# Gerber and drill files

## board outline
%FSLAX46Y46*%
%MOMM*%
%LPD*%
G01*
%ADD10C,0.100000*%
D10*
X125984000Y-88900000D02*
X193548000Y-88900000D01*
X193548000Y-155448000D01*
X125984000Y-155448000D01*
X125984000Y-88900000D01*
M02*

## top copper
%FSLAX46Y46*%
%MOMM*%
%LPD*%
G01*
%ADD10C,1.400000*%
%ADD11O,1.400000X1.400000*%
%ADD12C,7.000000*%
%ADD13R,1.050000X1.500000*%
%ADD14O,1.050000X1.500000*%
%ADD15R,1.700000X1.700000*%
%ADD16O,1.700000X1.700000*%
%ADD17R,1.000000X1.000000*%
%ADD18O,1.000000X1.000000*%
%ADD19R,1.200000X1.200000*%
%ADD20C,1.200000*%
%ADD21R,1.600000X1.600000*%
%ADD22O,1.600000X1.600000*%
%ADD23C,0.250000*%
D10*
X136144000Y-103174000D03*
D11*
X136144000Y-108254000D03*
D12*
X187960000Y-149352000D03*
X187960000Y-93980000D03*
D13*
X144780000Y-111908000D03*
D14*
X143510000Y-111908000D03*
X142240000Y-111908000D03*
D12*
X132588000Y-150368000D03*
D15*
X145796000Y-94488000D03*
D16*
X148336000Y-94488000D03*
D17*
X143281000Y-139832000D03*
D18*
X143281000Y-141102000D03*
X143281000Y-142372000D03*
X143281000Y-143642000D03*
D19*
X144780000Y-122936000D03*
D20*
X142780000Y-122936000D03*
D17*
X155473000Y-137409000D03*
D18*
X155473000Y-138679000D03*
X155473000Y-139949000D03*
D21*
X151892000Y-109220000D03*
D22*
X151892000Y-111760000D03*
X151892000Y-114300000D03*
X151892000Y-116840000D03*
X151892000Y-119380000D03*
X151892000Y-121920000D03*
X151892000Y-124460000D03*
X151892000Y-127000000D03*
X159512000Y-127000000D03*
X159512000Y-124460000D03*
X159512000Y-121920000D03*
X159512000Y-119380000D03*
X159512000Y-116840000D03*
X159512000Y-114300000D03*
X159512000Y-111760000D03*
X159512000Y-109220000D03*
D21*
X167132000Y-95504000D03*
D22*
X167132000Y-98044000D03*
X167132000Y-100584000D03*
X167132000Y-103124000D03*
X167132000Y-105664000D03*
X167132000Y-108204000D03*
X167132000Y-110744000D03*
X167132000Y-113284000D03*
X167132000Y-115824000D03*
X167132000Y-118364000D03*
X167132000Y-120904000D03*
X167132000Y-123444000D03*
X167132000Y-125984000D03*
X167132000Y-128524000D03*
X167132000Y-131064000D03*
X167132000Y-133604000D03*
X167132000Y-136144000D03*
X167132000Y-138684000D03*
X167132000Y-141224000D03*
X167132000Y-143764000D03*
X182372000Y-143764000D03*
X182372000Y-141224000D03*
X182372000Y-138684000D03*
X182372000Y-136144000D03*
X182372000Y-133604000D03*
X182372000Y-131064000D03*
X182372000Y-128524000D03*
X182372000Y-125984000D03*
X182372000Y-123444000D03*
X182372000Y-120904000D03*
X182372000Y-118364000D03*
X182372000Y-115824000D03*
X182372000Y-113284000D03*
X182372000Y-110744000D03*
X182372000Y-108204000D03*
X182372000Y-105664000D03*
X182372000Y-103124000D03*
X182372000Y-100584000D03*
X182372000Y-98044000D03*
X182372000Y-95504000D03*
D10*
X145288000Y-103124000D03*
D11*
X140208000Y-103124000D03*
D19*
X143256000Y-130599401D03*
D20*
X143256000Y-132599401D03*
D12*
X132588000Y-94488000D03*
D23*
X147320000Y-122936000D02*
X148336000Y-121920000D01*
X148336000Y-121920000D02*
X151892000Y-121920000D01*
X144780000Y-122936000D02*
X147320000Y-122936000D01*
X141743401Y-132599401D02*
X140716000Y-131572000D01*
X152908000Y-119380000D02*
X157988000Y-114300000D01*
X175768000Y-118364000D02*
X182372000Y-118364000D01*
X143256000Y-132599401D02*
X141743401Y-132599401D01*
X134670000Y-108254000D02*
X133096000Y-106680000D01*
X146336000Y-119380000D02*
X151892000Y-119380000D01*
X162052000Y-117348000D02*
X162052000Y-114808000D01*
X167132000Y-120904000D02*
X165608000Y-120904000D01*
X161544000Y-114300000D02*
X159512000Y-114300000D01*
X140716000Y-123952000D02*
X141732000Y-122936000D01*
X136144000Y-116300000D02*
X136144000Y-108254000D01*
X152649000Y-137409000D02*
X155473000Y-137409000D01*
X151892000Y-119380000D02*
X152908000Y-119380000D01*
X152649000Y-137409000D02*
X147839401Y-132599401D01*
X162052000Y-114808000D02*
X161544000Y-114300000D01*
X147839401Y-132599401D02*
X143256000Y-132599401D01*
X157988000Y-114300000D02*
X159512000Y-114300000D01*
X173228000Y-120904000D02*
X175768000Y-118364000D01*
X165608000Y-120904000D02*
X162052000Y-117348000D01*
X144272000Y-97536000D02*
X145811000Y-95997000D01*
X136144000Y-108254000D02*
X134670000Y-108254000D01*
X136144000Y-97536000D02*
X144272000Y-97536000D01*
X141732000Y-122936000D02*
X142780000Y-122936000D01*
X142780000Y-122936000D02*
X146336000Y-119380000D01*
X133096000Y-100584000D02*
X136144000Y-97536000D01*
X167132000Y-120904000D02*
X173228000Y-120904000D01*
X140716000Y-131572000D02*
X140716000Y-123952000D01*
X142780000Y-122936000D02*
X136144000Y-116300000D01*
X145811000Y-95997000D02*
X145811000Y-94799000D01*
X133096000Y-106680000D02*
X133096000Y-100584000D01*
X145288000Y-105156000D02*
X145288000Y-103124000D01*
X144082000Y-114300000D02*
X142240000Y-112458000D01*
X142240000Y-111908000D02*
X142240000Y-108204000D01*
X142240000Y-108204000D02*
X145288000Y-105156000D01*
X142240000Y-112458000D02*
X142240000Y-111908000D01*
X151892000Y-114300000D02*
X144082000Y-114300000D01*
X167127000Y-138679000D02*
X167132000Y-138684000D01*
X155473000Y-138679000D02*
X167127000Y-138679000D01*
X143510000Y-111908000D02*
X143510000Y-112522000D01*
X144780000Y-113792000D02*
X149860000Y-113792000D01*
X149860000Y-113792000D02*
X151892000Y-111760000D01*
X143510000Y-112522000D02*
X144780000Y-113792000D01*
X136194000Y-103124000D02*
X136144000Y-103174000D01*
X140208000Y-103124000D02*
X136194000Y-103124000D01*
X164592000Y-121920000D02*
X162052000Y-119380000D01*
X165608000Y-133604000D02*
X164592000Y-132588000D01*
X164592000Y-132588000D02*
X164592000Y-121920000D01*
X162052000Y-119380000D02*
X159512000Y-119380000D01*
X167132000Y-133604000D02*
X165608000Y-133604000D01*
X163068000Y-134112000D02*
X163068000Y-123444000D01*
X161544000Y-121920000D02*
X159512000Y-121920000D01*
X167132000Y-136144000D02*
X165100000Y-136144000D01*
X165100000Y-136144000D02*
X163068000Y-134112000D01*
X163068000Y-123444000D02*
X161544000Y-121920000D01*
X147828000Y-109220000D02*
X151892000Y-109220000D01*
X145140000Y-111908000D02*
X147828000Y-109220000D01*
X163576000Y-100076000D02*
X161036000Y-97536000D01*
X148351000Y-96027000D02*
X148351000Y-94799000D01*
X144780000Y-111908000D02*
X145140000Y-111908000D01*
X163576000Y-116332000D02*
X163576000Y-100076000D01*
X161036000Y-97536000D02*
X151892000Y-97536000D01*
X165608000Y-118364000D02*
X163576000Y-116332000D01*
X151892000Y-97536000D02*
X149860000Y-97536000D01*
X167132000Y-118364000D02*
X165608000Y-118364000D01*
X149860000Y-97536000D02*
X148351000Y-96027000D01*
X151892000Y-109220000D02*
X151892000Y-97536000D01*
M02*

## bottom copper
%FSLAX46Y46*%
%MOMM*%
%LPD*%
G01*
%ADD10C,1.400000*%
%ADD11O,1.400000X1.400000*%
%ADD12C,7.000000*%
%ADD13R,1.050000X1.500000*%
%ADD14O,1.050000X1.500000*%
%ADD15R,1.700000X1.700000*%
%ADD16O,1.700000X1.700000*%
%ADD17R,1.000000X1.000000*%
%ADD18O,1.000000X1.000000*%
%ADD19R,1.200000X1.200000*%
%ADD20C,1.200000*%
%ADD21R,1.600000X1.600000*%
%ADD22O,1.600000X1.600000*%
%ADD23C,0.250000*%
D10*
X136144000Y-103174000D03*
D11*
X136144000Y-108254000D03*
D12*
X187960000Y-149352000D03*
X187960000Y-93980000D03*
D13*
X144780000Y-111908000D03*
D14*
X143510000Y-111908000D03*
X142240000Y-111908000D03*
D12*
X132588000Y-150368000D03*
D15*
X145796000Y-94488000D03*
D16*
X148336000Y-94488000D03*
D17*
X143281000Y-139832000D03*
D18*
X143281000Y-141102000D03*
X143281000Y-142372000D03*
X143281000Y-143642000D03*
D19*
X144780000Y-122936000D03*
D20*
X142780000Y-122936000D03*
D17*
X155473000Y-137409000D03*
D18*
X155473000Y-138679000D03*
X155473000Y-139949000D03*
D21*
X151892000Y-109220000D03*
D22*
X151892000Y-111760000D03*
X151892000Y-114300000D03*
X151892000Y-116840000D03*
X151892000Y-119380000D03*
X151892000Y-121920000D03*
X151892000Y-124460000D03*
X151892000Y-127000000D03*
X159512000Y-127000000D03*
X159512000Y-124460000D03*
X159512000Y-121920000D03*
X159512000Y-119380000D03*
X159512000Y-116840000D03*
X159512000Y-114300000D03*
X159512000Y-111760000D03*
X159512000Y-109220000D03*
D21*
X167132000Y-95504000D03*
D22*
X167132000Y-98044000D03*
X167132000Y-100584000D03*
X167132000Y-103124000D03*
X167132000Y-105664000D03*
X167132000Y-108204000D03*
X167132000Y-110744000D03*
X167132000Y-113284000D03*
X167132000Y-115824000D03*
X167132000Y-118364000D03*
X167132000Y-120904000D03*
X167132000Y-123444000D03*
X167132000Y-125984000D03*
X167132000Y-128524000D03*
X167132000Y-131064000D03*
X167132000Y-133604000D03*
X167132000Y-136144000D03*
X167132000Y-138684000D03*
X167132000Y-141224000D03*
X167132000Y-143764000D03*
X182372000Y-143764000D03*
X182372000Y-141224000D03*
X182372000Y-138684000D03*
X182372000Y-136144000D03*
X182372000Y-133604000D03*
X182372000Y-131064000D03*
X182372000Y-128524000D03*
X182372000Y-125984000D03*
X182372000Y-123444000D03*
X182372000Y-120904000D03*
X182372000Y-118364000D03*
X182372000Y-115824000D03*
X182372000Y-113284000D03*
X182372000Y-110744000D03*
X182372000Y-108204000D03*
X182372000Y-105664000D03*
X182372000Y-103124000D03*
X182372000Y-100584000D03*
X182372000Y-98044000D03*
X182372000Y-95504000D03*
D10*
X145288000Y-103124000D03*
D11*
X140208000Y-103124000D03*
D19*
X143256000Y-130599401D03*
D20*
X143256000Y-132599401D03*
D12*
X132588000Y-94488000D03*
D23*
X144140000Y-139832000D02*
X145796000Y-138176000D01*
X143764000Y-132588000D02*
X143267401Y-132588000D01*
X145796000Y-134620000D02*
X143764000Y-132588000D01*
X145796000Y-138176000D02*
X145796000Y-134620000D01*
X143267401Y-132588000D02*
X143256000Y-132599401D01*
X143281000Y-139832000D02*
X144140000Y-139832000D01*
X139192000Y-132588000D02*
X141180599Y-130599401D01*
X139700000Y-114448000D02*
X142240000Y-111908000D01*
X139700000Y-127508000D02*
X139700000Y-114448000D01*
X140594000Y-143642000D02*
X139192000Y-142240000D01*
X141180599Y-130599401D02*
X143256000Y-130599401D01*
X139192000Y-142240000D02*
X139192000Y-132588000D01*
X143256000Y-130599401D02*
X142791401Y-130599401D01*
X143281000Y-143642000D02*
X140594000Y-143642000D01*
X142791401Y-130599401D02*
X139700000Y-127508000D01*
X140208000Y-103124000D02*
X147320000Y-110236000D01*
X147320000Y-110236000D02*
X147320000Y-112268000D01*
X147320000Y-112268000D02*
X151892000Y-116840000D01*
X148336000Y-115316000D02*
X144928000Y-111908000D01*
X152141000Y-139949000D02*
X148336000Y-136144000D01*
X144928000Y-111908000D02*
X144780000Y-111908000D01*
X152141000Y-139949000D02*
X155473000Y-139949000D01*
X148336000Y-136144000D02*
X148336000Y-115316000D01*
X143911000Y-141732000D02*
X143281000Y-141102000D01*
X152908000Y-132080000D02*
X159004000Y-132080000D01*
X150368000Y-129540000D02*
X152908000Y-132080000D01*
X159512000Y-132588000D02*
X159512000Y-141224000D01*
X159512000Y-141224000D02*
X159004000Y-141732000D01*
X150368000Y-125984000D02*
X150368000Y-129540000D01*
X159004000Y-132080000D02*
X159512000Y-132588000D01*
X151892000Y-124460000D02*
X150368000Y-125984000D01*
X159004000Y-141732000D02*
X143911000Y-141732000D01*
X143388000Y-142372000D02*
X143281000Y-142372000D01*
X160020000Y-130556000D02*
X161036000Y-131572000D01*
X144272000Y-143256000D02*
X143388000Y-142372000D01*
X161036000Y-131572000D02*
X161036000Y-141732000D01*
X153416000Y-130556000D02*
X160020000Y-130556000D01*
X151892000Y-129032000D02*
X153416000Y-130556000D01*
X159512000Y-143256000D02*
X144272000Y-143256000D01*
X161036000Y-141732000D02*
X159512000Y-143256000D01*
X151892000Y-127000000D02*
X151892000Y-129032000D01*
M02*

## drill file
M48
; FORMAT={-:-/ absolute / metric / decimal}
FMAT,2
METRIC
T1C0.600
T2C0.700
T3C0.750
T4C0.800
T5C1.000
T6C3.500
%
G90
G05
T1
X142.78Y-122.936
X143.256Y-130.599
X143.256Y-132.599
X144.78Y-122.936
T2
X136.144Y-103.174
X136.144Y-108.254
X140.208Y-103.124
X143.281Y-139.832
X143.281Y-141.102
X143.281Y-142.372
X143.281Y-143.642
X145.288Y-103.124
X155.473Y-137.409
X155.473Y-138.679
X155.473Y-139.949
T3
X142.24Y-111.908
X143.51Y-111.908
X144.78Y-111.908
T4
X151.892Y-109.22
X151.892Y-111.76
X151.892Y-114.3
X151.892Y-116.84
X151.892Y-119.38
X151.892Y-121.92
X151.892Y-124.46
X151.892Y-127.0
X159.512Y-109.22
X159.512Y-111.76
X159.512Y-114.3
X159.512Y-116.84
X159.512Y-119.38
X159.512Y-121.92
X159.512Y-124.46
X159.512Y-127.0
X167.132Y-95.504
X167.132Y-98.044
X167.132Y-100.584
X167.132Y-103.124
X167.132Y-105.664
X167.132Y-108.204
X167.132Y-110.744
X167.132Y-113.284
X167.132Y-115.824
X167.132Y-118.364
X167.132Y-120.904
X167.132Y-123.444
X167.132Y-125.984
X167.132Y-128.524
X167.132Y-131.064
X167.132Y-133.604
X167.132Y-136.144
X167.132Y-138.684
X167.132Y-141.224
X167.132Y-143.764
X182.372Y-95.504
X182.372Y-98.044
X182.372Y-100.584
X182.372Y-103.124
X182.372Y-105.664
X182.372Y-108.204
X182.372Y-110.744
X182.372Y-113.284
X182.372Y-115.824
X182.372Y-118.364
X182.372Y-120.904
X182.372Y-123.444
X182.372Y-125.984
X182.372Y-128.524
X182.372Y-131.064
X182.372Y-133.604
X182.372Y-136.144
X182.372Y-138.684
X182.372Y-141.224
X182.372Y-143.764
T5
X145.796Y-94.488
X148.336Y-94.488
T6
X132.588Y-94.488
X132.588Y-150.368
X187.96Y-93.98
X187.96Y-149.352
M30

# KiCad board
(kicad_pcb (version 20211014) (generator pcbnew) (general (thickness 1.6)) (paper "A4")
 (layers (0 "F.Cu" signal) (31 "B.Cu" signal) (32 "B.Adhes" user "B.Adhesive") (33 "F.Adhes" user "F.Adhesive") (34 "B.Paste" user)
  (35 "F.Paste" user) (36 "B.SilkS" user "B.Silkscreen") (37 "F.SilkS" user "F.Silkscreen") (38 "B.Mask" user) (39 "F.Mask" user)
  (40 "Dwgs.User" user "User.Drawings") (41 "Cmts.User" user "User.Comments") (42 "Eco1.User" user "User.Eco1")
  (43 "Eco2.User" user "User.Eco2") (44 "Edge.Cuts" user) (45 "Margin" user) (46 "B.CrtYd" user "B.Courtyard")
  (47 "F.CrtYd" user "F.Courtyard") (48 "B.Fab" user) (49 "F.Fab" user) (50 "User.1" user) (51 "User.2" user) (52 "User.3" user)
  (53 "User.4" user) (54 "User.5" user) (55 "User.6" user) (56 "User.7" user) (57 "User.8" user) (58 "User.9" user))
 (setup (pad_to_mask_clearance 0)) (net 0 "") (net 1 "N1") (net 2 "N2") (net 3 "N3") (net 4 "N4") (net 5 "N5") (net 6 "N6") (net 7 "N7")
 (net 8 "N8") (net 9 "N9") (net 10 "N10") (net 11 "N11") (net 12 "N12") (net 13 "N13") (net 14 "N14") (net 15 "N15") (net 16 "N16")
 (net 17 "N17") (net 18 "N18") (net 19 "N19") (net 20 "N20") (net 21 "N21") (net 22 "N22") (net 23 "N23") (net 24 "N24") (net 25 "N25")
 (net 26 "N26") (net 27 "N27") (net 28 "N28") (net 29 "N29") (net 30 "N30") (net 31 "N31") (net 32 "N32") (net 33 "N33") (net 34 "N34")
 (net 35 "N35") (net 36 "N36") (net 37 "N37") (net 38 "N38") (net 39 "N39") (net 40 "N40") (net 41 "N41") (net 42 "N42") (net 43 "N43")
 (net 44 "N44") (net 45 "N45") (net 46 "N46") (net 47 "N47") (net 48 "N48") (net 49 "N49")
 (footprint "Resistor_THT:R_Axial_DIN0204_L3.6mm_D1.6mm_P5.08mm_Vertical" (layer "F.Cu") (at 136.144 103.174 -90)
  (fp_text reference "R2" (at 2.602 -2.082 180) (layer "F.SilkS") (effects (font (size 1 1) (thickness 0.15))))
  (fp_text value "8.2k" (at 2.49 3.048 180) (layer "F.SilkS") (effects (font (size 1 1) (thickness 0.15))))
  (pad "1" thru_hole circle (at 0 0 270) (size 1.4 1.4) (drill 0.7) (layers *.Cu *.Mask) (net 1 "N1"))
  (pad "2" thru_hole oval (at 5.08 0 270) (size 1.4 1.4) (drill 0.7) (layers *.Cu *.Mask) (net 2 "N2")))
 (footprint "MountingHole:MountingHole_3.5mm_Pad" (layer "F.Cu") (at 187.96 149.352)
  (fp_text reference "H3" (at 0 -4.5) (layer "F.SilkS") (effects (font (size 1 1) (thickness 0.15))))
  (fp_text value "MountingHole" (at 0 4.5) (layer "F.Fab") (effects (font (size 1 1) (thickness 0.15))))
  (pad "1" thru_hole circle (at 0 0) (size 7 7) (drill 3.5) (layers *.Cu *.Mask)))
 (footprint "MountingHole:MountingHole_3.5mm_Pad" (layer "F.Cu") (at 187.96 93.98)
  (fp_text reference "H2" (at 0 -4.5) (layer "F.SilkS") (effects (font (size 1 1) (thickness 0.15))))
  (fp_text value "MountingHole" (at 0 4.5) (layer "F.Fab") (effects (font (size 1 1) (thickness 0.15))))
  (pad "1" thru_hole circle (at 0 0) (size 7 7) (drill 3.5) (layers *.Cu *.Mask)))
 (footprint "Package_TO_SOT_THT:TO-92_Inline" (layer "F.Cu") (at 144.78 111.908 180)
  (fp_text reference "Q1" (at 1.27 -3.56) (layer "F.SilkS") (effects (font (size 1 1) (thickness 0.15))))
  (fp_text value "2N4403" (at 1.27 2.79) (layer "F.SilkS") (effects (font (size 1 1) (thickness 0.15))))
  (pad "1" thru_hole rect (at 0 0 180) (size 1.05 1.5) (drill 0.75) (layers *.Cu *.Mask) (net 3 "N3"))
  (pad "2" thru_hole oval (at 1.27 0 180) (size 1.05 1.5) (drill 0.75) (layers *.Cu *.Mask) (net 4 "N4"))
  (pad "3" thru_hole oval (at 2.54 0 180) (size 1.05 1.5) (drill 0.75) (layers *.Cu *.Mask) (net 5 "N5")))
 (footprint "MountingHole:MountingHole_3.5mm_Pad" (layer "F.Cu") (at 132.588 150.368)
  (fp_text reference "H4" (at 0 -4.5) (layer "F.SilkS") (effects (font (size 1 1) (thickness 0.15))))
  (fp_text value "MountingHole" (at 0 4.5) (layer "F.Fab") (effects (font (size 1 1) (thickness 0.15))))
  (pad "1" thru_hole circle (at 0 0) (size 7 7) (drill 3.5) (layers *.Cu *.Mask)))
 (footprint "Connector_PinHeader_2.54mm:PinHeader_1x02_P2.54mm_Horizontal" (layer "F.Cu") (at 145.796 94.488 90)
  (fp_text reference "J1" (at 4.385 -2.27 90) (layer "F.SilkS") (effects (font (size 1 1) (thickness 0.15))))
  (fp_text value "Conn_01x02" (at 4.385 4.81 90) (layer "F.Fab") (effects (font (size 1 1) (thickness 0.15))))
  (pad "1" thru_hole rect (at 0 0 90) (size 1.7 1.7) (drill 1) (layers *.Cu *.Mask) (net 2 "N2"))
  (pad "2" thru_hole oval (at 0 2.54 90) (size 1.7 1.7) (drill 1) (layers *.Cu *.Mask) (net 3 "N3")))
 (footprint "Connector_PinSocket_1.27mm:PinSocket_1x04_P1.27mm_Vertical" (layer "F.Cu") (at 143.281 139.832)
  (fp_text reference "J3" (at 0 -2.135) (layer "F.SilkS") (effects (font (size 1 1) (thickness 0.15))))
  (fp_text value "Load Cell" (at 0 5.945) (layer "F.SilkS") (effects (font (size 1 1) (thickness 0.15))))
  (pad "1" thru_hole rect (at 0 0) (size 1 1) (drill 0.7) (layers *.Cu *.Mask) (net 2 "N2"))
  (pad "2" thru_hole oval (at 0 1.27) (size 1 1) (drill 0.7) (layers *.Cu *.Mask) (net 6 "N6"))
  (pad "3" thru_hole oval (at 0 2.54) (size 1 1) (drill 0.7) (layers *.Cu *.Mask) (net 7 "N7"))
  (pad "4" thru_hole oval (at 0 3.81) (size 1 1) (drill 0.7) (layers *.Cu *.Mask) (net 5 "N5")))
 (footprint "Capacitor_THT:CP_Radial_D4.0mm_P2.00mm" (layer "F.Cu") (at 144.78 122.936 180)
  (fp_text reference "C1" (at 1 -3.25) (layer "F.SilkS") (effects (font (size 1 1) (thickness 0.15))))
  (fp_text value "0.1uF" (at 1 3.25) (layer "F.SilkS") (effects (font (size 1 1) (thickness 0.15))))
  (pad "1" thru_hole rect (at 0 0 180) (size 1.2 1.2) (drill 0.6) (layers *.Cu *.Mask) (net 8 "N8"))
  (pad "2" thru_hole circle (at 2 0 180) (size 1.2 1.2) (drill 0.6) (layers *.Cu *.Mask) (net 2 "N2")))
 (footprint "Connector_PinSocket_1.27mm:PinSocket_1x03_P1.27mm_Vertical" (layer "F.Cu") (at 155.473 137.409)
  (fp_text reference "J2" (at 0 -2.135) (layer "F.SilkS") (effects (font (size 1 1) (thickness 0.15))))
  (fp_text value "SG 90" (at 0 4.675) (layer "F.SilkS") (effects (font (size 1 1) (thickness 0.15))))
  (pad "1" thru_hole rect (at 0 0) (size 1 1) (drill 0.7) (layers *.Cu *.Mask) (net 2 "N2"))
  (pad "2" thru_hole oval (at 0 1.27) (size 1 1) (drill 0.7) (layers *.Cu *.Mask) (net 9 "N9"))
  (pad "3" thru_hole oval (at 0 2.54) (size 1 1) (drill 0.7) (layers *.Cu *.Mask) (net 3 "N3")))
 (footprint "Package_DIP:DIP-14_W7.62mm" (layer "F.Cu") (at 151.892 109.22)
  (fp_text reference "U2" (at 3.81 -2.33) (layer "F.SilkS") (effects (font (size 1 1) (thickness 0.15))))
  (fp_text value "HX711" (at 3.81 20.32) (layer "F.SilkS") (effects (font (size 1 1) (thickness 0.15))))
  (pad "1" thru_hole rect (at 0 0) (size 1.6 1.6) (drill 0.8) (layers *.Cu *.Mask) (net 3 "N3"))
  (pad "2" thru_hole oval (at 0 2.54) (size 1.6 1.6) (drill 0.8) (layers *.Cu *.Mask) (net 4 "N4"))
  (pad "3" thru_hole oval (at 0 5.08) (size 1.6 1.6) (drill 0.8) (layers *.Cu *.Mask) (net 5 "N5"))
  (pad "4" thru_hole oval (at 0 7.62) (size 1.6 1.6) (drill 0.8) (layers *.Cu *.Mask) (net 1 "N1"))
  (pad "5" thru_hole oval (at 0 10.16) (size 1.6 1.6) (drill 0.8) (layers *.Cu *.Mask) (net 2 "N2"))
  (pad "6" thru_hole oval (at 0 12.7) (size 1.6 1.6) (drill 0.8) (layers *.Cu *.Mask) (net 8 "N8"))
  (pad "7" thru_hole oval (at 0 15.24) (size 1.6 1.6) (drill 0.8) (layers *.Cu *.Mask) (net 6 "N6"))
  (pad "8" thru_hole oval (at 0 17.78) (size 1.6 1.6) (drill 0.8) (layers *.Cu *.Mask) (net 7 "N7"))
  (pad "9" thru_hole oval (at 7.62 17.78) (size 1.6 1.6) (drill 0.8) (layers *.Cu *.Mask) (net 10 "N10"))
  (pad "10" thru_hole oval (at 7.62 15.24) (size 1.6 1.6) (drill 0.8) (layers *.Cu *.Mask) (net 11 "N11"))
  (pad "11" thru_hole oval (at 7.62 12.7) (size 1.6 1.6) (drill 0.8) (layers *.Cu *.Mask) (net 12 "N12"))
  (pad "12" thru_hole oval (at 7.62 10.16) (size 1.6 1.6) (drill 0.8) (layers *.Cu *.Mask) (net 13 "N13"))
  (pad "13" thru_hole oval (at 7.62 7.62) (size 1.6 1.6) (drill 0.8) (layers *.Cu *.Mask) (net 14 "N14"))
  (pad "14" thru_hole oval (at 7.62 5.08) (size 1.6 1.6) (drill 0.8) (layers *.Cu *.Mask) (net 2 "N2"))
  (pad "15" thru_hole oval (at 7.62 2.54) (size 1.6 1.6) (drill 0.8) (layers *.Cu *.Mask) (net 2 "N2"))
  (pad "16" thru_hole oval (at 7.62 0) (size 1.6 1.6) (drill 0.8) (layers *.Cu *.Mask) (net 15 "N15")))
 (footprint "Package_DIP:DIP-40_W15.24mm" (layer "F.Cu") (at 167.132 95.504)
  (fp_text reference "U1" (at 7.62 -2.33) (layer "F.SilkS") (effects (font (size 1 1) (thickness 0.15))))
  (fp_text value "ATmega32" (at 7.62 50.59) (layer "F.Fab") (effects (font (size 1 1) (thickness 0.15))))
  (pad "1" thru_hole rect (at 0 0) (size 1.6 1.6) (drill 0.8) (layers *.Cu *.Mask) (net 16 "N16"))
  (pad "2" thru_hole oval (at 0 2.54) (size 1.6 1.6) (drill 0.8) (layers *.Cu *.Mask) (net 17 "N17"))
  (pad "3" thru_hole oval (at 0 5.08) (size 1.6 1.6) (drill 0.8) (layers *.Cu *.Mask) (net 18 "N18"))
  (pad "4" thru_hole oval (at 0 7.62) (size 1.6 1.6) (drill 0.8) (layers *.Cu *.Mask) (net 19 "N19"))
  (pad "5" thru_hole oval (at 0 10.16) (size 1.6 1.6) (drill 0.8) (layers *.Cu *.Mask) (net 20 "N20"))
  (pad "6" thru_hole oval (at 0 12.7) (size 1.6 1.6) (drill 0.8) (layers *.Cu *.Mask) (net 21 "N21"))
  (pad "7" thru_hole oval (at 0 15.24) (size 1.6 1.6) (drill 0.8) (layers *.Cu *.Mask) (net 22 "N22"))
  (pad "8" thru_hole oval (at 0 17.78) (size 1.6 1.6) (drill 0.8) (layers *.Cu *.Mask) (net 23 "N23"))
  (pad "9" thru_hole oval (at 0 20.32) (size 1.6 1.6) (drill 0.8) (layers *.Cu *.Mask) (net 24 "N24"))
  (pad "10" thru_hole oval (at 0 22.86) (size 1.6 1.6) (drill 0.8) (layers *.Cu *.Mask) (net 3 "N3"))
  (pad "11" thru_hole oval (at 0 25.4) (size 1.6 1.6) (drill 0.8) (layers *.Cu *.Mask) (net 2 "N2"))
  (pad "12" thru_hole oval (at 0 27.94) (size 1.6 1.6) (drill 0.8) (layers *.Cu *.Mask) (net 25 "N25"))
  (pad "13" thru_hole oval (at 0 30.48) (size 1.6 1.6) (drill 0.8) (layers *.Cu *.Mask) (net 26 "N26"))
  (pad "14" thru_hole oval (at 0 33.02) (size 1.6 1.6) (drill 0.8) (layers *.Cu *.Mask) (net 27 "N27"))
  (pad "15" thru_hole oval (at 0 35.56) (size 1.6 1.6) (drill 0.8) (layers *.Cu *.Mask) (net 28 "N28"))
  (pad "16" thru_hole oval (at 0 38.1) (size 1.6 1.6) (drill 0.8) (layers *.Cu *.Mask) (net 13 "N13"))
  (pad "17" thru_hole oval (at 0 40.64) (size 1.6 1.6) (drill 0.8) (layers *.Cu *.Mask) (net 12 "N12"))
  (pad "18" thru_hole oval (at 0 43.18) (size 1.6 1.6) (drill 0.8) (layers *.Cu *.Mask) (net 9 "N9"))
  (pad "19" thru_hole oval (at 0 45.72) (size 1.6 1.6) (drill 0.8) (layers *.Cu *.Mask) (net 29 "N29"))
  (pad "20" thru_hole oval (at 0 48.26) (size 1.6 1.6) (drill 0.8) (layers *.Cu *.Mask) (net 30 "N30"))
  (pad "21" thru_hole oval (at 15.24 48.26) (size 1.6 1.6) (drill 0.8) (layers *.Cu *.Mask) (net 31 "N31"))
  (pad "22" thru_hole oval (at 15.24 45.72) (size 1.6 1.6) (drill 0.8) (layers *.Cu *.Mask) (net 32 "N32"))
  (pad "23" thru_hole oval (at 15.24 43.18) (size 1.6 1.6) (drill 0.8) (layers *.Cu *.Mask) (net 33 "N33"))
  (pad "24" thru_hole oval (at 15.24 40.64) (size 1.6 1.6) (drill 0.8) (layers *.Cu *.Mask) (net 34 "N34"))
  (pad "25" thru_hole oval (at 15.24 38.1) (size 1.6 1.6) (drill 0.8) (layers *.Cu *.Mask) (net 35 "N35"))
  (pad "26" thru_hole oval (at 15.24 35.56) (size 1.6 1.6) (drill 0.8) (layers *.Cu *.Mask) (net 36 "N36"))
  (pad "27" thru_hole oval (at 15.24 33.02) (size 1.6 1.6) (drill 0.8) (layers *.Cu *.Mask) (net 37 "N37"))
  (pad "28" thru_hole oval (at 15.24 30.48) (size 1.6 1.6) (drill 0.8) (layers *.Cu *.Mask) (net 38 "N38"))
  (pad "29" thru_hole oval (at 15.24 27.94) (size 1.6 1.6) (drill 0.8) (layers *.Cu *.Mask) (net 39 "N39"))
  (pad "30" thru_hole oval (at 15.24 25.4) (size 1.6 1.6) (drill 0.8) (layers *.Cu *.Mask) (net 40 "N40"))
  (pad "31" thru_hole oval (at 15.24 22.86) (size 1.6 1.6) (drill 0.8) (layers *.Cu *.Mask) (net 2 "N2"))
  (pad "32" thru_hole oval (at 15.24 20.32) (size 1.6 1.6) (drill 0.8) (layers *.Cu *.Mask) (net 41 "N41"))
  (pad "33" thru_hole oval (at 15.24 17.78) (size 1.6 1.6) (drill 0.8) (layers *.Cu *.Mask) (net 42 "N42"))
  (pad "34" thru_hole oval (at 15.24 15.24) (size 1.6 1.6) (drill 0.8) (layers *.Cu *.Mask) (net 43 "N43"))
  (pad "35" thru_hole oval (at 15.24 12.7) (size 1.6 1.6) (drill 0.8) (layers *.Cu *.Mask) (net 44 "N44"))
  (pad "36" thru_hole oval (at 15.24 10.16) (size 1.6 1.6) (drill 0.8) (layers *.Cu *.Mask) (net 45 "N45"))
  (pad "37" thru_hole oval (at 15.24 7.62) (size 1.6 1.6) (drill 0.8) (layers *.Cu *.Mask) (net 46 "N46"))
  (pad "38" thru_hole oval (at 15.24 5.08) (size 1.6 1.6) (drill 0.8) (layers *.Cu *.Mask) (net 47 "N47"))
  (pad "39" thru_hole oval (at 15.24 2.54) (size 1.6 1.6) (drill 0.8) (layers *.Cu *.Mask) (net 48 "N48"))
  (pad "40" thru_hole oval (at 15.24 0) (size 1.6 1.6) (drill 0.8) (layers *.Cu *.Mask) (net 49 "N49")))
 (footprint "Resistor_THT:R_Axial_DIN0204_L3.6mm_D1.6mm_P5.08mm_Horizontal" (layer "F.Cu") (at 145.288 103.124 180)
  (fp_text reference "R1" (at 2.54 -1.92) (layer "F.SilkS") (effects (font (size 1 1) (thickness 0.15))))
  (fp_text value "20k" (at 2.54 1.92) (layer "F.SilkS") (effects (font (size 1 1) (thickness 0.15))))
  (pad "1" thru_hole circle (at 0 0 180) (size 1.4 1.4) (drill 0.7) (layers *.Cu *.Mask) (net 5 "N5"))
  (pad "2" thru_hole oval (at 5.08 0 180) (size 1.4 1.4) (drill 0.7) (layers *.Cu *.Mask) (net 1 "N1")))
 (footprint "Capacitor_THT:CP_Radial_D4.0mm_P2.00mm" (layer "F.Cu") (at 143.256 130.599401 -90)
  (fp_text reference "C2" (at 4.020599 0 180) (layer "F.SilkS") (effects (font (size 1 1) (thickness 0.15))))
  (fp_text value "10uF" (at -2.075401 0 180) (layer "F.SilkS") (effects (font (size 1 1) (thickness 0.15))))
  (pad "1" thru_hole rect (at 0 0 270) (size 1.2 1.2) (drill 0.6) (layers *.Cu *.Mask) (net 5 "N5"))
  (pad "2" thru_hole circle (at 2 0 270) (size 1.2 1.2) (drill 0.6) (layers *.Cu *.Mask) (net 2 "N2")))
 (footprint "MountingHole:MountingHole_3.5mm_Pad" (layer "F.Cu") (at 132.588 94.488)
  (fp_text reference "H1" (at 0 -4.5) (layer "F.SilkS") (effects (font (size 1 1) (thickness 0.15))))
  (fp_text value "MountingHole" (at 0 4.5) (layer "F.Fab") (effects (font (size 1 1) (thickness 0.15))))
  (pad "1" thru_hole circle (at 0 0) (size 7 7) (drill 3.5) (layers *.Cu *.Mask)))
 (gr_rect (start 125.984 88.9) (end 193.548 155.448) (layer "Edge.Cuts") (width 0.1) (fill none))
 (segment (start 147.32 122.936) (end 148.336 121.92) (width 0.25) (layer "F.Cu") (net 8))
 (segment (start 148.336 121.92) (end 151.892 121.92) (width 0.25) (layer "F.Cu") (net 8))
 (segment (start 144.78 122.936) (end 147.32 122.936) (width 0.25) (layer "F.Cu") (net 8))
 (segment (start 141.743401 132.599401) (end 140.716 131.572) (width 0.25) (layer "F.Cu") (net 2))
 (segment (start 152.908 119.38) (end 157.988 114.3) (width 0.25) (layer "F.Cu") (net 2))
 (segment (start 175.768 118.364) (end 182.372 118.364) (width 0.25) (layer "F.Cu") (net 2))
 (segment (start 143.256 132.599401) (end 141.743401 132.599401) (width 0.25) (layer "F.Cu") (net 2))
 (segment (start 134.67 108.254) (end 133.096 106.68) (width 0.25) (layer "F.Cu") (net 2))
 (segment (start 146.336 119.38) (end 151.892 119.38) (width 0.25) (layer "F.Cu") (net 2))
 (segment (start 162.052 117.348) (end 162.052 114.808) (width 0.25) (layer "F.Cu") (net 2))
 (segment (start 167.132 120.904) (end 165.608 120.904) (width 0.25) (layer "F.Cu") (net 2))
 (segment (start 161.544 114.3) (end 159.512 114.3) (width 0.25) (layer "F.Cu") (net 2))
 (segment (start 140.716 123.952) (end 141.732 122.936) (width 0.25) (layer "F.Cu") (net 2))
 (segment (start 136.144 116.3) (end 136.144 108.254) (width 0.25) (layer "F.Cu") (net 2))
 (segment (start 152.649 137.409) (end 155.473 137.409) (width 0.25) (layer "F.Cu") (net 2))
 (segment (start 151.892 119.38) (end 152.908 119.38) (width 0.25) (layer "F.Cu") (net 2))
 (segment (start 152.649 137.409) (end 147.839401 132.599401) (width 0.25) (layer "F.Cu") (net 2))
 (segment (start 162.052 114.808) (end 161.544 114.3) (width 0.25) (layer "F.Cu") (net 2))
 (segment (start 147.839401 132.599401) (end 143.256 132.599401) (width 0.25) (layer "F.Cu") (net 2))
 (segment (start 157.988 114.3) (end 159.512 114.3) (width 0.25) (layer "F.Cu") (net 2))
 (segment (start 173.228 120.904) (end 175.768 118.364) (width 0.25) (layer "F.Cu") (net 2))
 (segment (start 165.608 120.904) (end 162.052 117.348) (width 0.25) (layer "F.Cu") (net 2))
 (segment (start 144.272 97.536) (end 145.811 95.997) (width 0.25) (layer "F.Cu") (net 2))
 (segment (start 136.144 108.254) (end 134.67 108.254) (width 0.25) (layer "F.Cu") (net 2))
 (segment (start 136.144 97.536) (end 144.272 97.536) (width 0.25) (layer "F.Cu") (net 2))
 (segment (start 141.732 122.936) (end 142.78 122.936) (width 0.25) (layer "F.Cu") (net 2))
 (segment (start 142.78 122.936) (end 146.336 119.38) (width 0.25) (layer "F.Cu") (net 2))
 (segment (start 133.096 100.584) (end 136.144 97.536) (width 0.25) (layer "F.Cu") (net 2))
 (segment (start 167.132 120.904) (end 173.228 120.904) (width 0.25) (layer "F.Cu") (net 2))
 (segment (start 140.716 131.572) (end 140.716 123.952) (width 0.25) (layer "F.Cu") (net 2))
 (segment (start 142.78 122.936) (end 136.144 116.3) (width 0.25) (layer "F.Cu") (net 2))
 (segment (start 145.811 95.997) (end 145.811 94.799) (width 0.25) (layer "F.Cu") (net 2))
 (segment (start 133.096 106.68) (end 133.096 100.584) (width 0.25) (layer "F.Cu") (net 2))
 (segment (start 144.14 139.832) (end 145.796 138.176) (width 0.25) (layer "B.Cu") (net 2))
 (segment (start 143.764 132.588) (end 143.267401 132.588) (width 0.25) (layer "B.Cu") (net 2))
 (segment (start 145.796 134.62) (end 143.764 132.588) (width 0.25) (layer "B.Cu") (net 2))
 (segment (start 145.796 138.176) (end 145.796 134.62) (width 0.25) (layer "B.Cu") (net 2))
 (segment (start 143.267401 132.588) (end 143.256 132.599401) (width 0.25) (layer "B.Cu") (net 2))
 (segment (start 143.281 139.832) (end 144.14 139.832) (width 0.25) (layer "B.Cu") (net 2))
 (segment (start 145.288 105.156) (end 145.288 103.124) (width 0.25) (layer "F.Cu") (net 5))
 (segment (start 144.082 114.3) (end 142.24 112.458) (width 0.25) (layer "F.Cu") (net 5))
 (segment (start 142.24 111.908) (end 142.24 108.204) (width 0.25) (layer "F.Cu") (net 5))
 (segment (start 142.24 108.204) (end 145.288 105.156) (width 0.25) (layer "F.Cu") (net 5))
 (segment (start 142.24 112.458) (end 142.24 111.908) (width 0.25) (layer "F.Cu") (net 5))
 (segment (start 151.892 114.3) (end 144.082 114.3) (width 0.25) (layer "F.Cu") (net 5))
 (segment (start 139.192 132.588) (end 141.180599 130.599401) (width 0.25) (layer "B.Cu") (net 5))
 (segment (start 139.7 114.448) (end 142.24 111.908) (width 0.25) (layer "B.Cu") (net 5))
 (segment (start 139.7 127.508) (end 139.7 114.448) (width 0.25) (layer "B.Cu") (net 5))
 (segment (start 140.594 143.642) (end 139.192 142.24) (width 0.25) (layer "B.Cu") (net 5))
 (segment (start 141.180599 130.599401) (end 143.256 130.599401) (width 0.25) (layer "B.Cu") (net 5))
 (segment (start 139.192 142.24) (end 139.192 132.588) (width 0.25) (layer "B.Cu") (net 5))
 (segment (start 143.256 130.599401) (end 142.791401 130.599401) (width 0.25) (layer "B.Cu") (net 5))
 (segment (start 143.281 143.642) (end 140.594 143.642) (width 0.25) (layer "B.Cu") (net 5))
 (segment (start 142.791401 130.599401) (end 139.7 127.508) (width 0.25) (layer "B.Cu") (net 5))
 (segment (start 167.127 138.679) (end 167.132 138.684) (width 0.25) (layer "F.Cu") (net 9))
 (segment (start 155.473 138.679) (end 167.127 138.679) (width 0.25) (layer "F.Cu") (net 9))
 (segment (start 143.51 111.908) (end 143.51 112.522) (width 0.25) (layer "F.Cu") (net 4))
 (segment (start 144.78 113.792) (end 149.86 113.792) (width 0.25) (layer "F.Cu") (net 4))
 (segment (start 149.86 113.792) (end 151.892 111.76) (width 0.25) (layer "F.Cu") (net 4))
 (segment (start 143.51 112.522) (end 144.78 113.792) (width 0.25) (layer "F.Cu") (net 4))
 (segment (start 136.194 103.124) (end 136.144 103.174) (width 0.25) (layer "F.Cu") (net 1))
 (segment (start 140.208 103.124) (end 136.194 103.124) (width 0.25) (layer "F.Cu") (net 1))
 (segment (start 140.208 103.124) (end 147.32 110.236) (width 0.25) (layer "B.Cu") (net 1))
 (segment (start 147.32 110.236) (end 147.32 112.268) (width 0.25) (layer "B.Cu") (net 1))
 (segment (start 147.32 112.268) (end 151.892 116.84) (width 0.25) (layer "B.Cu") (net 1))
 (segment (start 164.592 121.92) (end 162.052 119.38) (width 0.25) (layer "F.Cu") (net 13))
 (segment (start 165.608 133.604) (end 164.592 132.588) (width 0.25) (layer "F.Cu") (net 13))
 (segment (start 164.592 132.588) (end 164.592 121.92) (width 0.25) (layer "F.Cu") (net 13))
 (segment (start 162.052 119.38) (end 159.512 119.38) (width 0.25) (layer "F.Cu") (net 13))
 (segment (start 167.132 133.604) (end 165.608 133.604) (width 0.25) (layer "F.Cu") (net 13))
 (segment (start 163.068 134.112) (end 163.068 123.444) (width 0.25) (layer "F.Cu") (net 12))
 (segment (start 161.544 121.92) (end 159.512 121.92) (width 0.25) (layer "F.Cu") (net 12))
 (segment (start 167.132 136.144) (end 165.1 136.144) (width 0.25) (layer "F.Cu") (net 12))
 (segment (start 165.1 136.144) (end 163.068 134.112) (width 0.25) (layer "F.Cu") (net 12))
 (segment (start 163.068 123.444) (end 161.544 121.92) (width 0.25) (layer "F.Cu") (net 12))
 (segment (start 147.828 109.22) (end 151.892 109.22) (width 0.25) (layer "F.Cu") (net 3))
 (segment (start 145.14 111.908) (end 147.828 109.22) (width 0.25) (layer "F.Cu") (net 3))
 (segment (start 163.576 100.076) (end 161.036 97.536) (width 0.25) (layer "F.Cu") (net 3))
 (segment (start 148.351 96.027) (end 148.351 94.799) (width 0.25) (layer "F.Cu") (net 3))
 (segment (start 144.78 111.908) (end 145.14 111.908) (width 0.25) (layer "F.Cu") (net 3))
 (segment (start 163.576 116.332) (end 163.576 100.076) (width 0.25) (layer "F.Cu") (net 3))
 (segment (start 161.036 97.536) (end 151.892 97.536) (width 0.25) (layer "F.Cu") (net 3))
 (segment (start 165.608 118.364) (end 163.576 116.332) (width 0.25) (layer "F.Cu") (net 3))
 (segment (start 151.892 97.536) (end 149.86 97.536) (width 0.25) (layer "F.Cu") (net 3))
 (segment (start 167.132 118.364) (end 165.608 118.364) (width 0.25) (layer "F.Cu") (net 3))
 (segment (start 149.86 97.536) (end 148.351 96.027) (width 0.25) (layer "F.Cu") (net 3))
 (segment (start 151.892 109.22) (end 151.892 97.536) (width 0.25) (layer "F.Cu") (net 3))
 (segment (start 148.336 115.316) (end 144.928 111.908) (width 0.25) (layer "B.Cu") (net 3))
 (segment (start 152.141 139.949) (end 148.336 136.144) (width 0.25) (layer "B.Cu") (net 3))
 (segment (start 144.928 111.908) (end 144.78 111.908) (width 0.25) (layer "B.Cu") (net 3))
 (segment (start 152.141 139.949) (end 155.473 139.949) (width 0.25) (layer "B.Cu") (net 3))
 (segment (start 148.336 136.144) (end 148.336 115.316) (width 0.25) (layer "B.Cu") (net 3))
 (segment (start 143.911 141.732) (end 143.281 141.102) (width 0.25) (layer "B.Cu") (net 6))
 (segment (start 152.908 132.08) (end 159.004 132.08) (width 0.25) (layer "B.Cu") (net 6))
 (segment (start 150.368 129.54) (end 152.908 132.08) (width 0.25) (layer "B.Cu") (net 6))
 (segment (start 159.512 132.588) (end 159.512 141.224) (width 0.25) (layer "B.Cu") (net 6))
 (segment (start 159.512 141.224) (end 159.004 141.732) (width 0.25) (layer "B.Cu") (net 6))
 (segment (start 150.368 125.984) (end 150.368 129.54) (width 0.25) (layer "B.Cu") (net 6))
 (segment (start 159.004 132.08) (end 159.512 132.588) (width 0.25) (layer "B.Cu") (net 6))
 (segment (start 151.892 124.46) (end 150.368 125.984) (width 0.25) (layer "B.Cu") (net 6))
 (segment (start 159.004 141.732) (end 143.911 141.732) (width 0.25) (layer "B.Cu") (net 6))
 (segment (start 143.388 142.372) (end 143.281 142.372) (width 0.25) (layer "B.Cu") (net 7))
 (segment (start 160.02 130.556) (end 161.036 131.572) (width 0.25) (layer "B.Cu") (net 7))
 (segment (start 144.272 143.256) (end 143.388 142.372) (width 0.25) (layer "B.Cu") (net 7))
 (segment (start 161.036 131.572) (end 161.036 141.732) (width 0.25) (layer "B.Cu") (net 7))
 (segment (start 153.416 130.556) (end 160.02 130.556) (width 0.25) (layer "B.Cu") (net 7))
 (segment (start 151.892 129.032) (end 153.416 130.556) (width 0.25) (layer "B.Cu") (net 7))
 (segment (start 159.512 143.256) (end 144.272 143.256) (width 0.25) (layer "B.Cu") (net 7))
 (segment (start 161.036 141.732) (end 159.512 143.256) (width 0.25) (layer "B.Cu") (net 7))
 (segment (start 151.892 127) (end 151.892 129.032) (width 0.25) (layer "B.Cu") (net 7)))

